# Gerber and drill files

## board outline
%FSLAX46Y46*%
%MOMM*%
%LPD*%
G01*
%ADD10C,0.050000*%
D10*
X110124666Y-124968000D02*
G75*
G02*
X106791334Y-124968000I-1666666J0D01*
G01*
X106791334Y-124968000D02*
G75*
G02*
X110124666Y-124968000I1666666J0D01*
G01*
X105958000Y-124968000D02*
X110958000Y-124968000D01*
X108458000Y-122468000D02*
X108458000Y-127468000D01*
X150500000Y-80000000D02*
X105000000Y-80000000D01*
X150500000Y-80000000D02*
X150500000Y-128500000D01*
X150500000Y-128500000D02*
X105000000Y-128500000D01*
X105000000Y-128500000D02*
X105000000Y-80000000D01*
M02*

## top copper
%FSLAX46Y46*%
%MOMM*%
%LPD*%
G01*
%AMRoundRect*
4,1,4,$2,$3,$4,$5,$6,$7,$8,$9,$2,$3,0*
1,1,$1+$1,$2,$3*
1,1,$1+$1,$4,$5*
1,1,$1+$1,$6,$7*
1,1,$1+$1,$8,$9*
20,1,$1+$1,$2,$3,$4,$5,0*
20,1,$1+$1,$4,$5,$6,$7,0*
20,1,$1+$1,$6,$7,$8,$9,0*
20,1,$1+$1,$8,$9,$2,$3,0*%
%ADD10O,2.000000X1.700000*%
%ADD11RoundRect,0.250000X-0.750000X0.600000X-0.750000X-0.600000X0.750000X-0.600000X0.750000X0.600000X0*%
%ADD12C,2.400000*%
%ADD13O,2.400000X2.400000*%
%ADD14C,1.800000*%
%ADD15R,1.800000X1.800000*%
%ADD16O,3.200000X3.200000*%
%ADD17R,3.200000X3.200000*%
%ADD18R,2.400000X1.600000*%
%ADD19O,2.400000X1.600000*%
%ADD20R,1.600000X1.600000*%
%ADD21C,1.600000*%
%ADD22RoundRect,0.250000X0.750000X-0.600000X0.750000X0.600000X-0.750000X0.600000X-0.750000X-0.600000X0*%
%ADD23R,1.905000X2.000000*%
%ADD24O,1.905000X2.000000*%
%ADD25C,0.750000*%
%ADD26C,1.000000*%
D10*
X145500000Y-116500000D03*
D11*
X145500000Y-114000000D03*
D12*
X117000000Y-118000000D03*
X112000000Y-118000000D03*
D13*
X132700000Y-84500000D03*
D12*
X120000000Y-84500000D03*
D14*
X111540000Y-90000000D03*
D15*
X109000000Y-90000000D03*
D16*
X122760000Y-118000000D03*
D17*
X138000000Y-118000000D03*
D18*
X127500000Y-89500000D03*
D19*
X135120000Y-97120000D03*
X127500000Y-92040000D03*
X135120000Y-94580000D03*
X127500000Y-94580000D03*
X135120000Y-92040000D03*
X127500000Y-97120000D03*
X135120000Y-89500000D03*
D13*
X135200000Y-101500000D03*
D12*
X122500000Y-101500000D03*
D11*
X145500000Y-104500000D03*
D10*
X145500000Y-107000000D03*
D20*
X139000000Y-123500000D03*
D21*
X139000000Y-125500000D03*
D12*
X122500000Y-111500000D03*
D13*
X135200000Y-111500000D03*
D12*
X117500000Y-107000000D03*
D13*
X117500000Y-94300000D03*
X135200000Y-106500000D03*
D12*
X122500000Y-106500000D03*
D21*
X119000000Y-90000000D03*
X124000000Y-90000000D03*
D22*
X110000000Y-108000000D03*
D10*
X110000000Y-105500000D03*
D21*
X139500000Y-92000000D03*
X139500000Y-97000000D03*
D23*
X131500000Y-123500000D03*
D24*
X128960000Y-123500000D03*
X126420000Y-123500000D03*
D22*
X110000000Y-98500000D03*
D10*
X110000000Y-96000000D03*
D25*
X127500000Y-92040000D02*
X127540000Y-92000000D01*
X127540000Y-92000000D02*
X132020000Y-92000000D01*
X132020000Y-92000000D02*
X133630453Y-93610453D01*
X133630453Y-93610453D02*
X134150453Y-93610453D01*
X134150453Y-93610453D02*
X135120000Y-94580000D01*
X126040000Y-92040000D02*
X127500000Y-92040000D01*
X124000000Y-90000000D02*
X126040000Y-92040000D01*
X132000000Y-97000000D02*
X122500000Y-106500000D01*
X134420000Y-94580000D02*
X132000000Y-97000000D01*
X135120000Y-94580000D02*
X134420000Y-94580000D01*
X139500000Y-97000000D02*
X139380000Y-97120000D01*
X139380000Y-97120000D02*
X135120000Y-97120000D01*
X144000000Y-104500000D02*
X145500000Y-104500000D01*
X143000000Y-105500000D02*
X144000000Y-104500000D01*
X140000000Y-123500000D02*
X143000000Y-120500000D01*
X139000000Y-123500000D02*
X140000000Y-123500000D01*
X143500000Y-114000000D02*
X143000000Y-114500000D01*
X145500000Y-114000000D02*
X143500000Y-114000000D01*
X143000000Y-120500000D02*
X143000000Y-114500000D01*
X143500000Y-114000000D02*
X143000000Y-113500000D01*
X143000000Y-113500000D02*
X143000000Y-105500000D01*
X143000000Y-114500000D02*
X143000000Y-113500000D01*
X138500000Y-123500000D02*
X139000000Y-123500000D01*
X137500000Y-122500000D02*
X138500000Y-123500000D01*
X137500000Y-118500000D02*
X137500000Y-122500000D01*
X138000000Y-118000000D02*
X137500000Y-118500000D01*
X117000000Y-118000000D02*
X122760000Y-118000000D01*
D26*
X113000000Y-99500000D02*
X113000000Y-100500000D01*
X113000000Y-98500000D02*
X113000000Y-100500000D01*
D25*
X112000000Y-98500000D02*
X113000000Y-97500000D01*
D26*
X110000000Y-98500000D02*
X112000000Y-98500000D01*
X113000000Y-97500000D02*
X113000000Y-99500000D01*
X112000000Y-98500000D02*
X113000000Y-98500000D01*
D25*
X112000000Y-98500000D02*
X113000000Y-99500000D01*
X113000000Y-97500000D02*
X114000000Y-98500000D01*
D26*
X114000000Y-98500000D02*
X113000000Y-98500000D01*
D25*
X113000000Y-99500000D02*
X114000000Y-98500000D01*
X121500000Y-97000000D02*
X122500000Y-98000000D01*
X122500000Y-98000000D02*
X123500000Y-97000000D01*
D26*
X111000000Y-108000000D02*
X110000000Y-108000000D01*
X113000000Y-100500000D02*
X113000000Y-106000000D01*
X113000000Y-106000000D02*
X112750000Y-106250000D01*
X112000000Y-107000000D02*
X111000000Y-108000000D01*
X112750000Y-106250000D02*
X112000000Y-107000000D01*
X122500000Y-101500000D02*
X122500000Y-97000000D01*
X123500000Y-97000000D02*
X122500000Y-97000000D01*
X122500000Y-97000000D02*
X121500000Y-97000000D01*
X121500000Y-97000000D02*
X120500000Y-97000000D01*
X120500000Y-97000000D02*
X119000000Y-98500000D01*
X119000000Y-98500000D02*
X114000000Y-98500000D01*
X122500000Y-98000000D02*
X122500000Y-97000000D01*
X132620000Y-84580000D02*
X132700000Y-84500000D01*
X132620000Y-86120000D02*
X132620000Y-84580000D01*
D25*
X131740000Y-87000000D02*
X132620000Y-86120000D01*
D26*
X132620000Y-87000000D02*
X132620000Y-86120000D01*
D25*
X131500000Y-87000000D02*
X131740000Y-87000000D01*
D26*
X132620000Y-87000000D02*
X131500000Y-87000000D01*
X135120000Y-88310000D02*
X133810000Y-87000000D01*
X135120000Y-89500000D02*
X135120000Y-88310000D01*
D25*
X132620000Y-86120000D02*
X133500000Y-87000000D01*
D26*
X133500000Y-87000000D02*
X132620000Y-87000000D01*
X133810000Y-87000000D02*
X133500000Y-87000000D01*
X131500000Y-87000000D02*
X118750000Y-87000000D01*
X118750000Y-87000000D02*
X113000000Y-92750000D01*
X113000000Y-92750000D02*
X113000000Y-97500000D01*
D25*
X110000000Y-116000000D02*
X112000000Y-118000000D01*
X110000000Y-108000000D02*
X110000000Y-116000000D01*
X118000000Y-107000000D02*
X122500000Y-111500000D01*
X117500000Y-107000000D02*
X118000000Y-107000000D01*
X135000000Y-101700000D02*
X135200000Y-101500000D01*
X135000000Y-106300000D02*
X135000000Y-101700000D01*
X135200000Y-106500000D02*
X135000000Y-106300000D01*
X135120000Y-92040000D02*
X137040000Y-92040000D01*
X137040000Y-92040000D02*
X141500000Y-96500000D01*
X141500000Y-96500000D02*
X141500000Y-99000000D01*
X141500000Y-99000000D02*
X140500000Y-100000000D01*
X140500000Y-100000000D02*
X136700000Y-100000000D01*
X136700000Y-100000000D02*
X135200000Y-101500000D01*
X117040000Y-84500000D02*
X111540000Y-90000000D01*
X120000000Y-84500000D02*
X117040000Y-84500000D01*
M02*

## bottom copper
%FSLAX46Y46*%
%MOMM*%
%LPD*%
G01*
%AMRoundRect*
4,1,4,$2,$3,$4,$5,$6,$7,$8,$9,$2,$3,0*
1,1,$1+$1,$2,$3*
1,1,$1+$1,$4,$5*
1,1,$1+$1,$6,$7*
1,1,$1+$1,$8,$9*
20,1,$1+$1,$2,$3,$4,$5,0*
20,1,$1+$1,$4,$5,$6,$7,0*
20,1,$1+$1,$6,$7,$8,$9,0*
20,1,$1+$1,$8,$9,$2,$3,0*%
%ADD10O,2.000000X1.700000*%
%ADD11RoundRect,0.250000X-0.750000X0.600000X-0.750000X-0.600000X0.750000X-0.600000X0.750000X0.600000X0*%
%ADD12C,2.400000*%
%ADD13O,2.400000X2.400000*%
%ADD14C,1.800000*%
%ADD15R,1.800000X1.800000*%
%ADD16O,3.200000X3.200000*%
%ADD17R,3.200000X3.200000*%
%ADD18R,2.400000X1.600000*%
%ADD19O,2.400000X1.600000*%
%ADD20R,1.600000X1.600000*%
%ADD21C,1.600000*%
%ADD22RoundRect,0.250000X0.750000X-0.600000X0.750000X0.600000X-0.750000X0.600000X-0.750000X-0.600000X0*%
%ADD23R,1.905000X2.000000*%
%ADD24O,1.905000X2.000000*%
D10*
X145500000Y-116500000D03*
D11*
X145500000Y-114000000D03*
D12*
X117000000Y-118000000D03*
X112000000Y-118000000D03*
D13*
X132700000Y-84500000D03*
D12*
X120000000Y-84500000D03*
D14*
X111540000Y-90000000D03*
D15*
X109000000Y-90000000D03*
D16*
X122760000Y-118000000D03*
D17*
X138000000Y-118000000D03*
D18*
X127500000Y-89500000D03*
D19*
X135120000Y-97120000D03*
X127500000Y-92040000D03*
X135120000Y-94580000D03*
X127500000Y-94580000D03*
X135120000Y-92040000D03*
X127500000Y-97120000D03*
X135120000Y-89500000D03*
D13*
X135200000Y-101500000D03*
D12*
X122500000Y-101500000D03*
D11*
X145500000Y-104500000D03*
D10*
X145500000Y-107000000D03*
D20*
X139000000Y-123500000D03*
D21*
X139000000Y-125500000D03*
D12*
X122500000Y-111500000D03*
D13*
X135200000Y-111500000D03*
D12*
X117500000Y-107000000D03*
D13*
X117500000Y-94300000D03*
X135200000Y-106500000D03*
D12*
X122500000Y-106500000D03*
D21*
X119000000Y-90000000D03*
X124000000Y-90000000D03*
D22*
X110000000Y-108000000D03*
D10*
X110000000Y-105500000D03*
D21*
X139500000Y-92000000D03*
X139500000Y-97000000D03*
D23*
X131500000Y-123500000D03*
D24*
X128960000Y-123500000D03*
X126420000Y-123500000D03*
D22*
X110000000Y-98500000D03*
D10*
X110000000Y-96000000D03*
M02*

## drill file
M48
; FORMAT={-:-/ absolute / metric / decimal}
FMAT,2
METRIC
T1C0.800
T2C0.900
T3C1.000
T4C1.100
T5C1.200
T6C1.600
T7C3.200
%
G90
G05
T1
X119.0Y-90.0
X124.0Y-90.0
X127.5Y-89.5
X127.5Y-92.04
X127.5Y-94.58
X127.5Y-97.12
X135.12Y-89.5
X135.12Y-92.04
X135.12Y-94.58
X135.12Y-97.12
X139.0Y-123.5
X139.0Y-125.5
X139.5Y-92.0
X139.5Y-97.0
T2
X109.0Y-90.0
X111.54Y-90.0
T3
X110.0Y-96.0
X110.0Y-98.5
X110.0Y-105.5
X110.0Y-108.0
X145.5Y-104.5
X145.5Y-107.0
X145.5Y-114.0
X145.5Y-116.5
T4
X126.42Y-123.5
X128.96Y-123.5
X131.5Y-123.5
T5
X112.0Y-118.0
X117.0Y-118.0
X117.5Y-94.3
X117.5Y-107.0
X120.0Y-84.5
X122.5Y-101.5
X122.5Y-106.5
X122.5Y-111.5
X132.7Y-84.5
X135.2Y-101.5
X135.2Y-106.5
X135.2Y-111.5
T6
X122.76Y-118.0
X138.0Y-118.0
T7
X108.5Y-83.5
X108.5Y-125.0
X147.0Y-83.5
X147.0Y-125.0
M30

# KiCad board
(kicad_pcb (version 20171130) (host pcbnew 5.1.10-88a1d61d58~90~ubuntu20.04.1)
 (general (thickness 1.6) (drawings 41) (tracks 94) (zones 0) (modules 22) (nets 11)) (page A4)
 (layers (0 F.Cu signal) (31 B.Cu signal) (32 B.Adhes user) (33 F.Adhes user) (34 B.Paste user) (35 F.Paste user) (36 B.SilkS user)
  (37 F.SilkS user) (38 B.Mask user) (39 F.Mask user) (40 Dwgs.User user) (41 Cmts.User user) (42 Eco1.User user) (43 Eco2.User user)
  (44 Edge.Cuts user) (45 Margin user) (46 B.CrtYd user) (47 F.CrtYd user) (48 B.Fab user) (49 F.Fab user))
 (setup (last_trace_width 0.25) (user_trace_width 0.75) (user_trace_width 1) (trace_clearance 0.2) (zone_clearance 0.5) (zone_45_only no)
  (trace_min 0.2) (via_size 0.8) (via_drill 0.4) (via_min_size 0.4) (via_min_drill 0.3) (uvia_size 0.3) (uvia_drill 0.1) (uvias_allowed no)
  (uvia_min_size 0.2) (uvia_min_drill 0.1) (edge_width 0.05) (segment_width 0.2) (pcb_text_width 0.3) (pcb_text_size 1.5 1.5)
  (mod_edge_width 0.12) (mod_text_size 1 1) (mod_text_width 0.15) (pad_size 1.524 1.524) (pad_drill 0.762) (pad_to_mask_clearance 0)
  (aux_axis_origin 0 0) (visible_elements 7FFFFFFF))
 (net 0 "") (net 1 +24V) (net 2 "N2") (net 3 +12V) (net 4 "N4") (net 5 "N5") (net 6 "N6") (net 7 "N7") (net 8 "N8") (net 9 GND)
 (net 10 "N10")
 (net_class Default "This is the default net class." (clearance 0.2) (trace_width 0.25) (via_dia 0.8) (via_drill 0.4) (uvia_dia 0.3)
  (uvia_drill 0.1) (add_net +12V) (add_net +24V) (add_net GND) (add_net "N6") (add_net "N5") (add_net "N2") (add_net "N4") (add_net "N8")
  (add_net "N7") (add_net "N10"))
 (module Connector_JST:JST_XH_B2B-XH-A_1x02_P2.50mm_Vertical (layer F.Cu) (at 145.5 114 270)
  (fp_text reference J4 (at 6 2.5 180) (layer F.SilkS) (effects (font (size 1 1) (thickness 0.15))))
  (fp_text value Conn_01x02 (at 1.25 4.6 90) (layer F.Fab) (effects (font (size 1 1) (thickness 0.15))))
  (pad 2 thru_hole oval (at 2.5 0 270) (size 1.7 2) (drill 1) (layers *.Cu *.Mask))
  (pad 1 thru_hole roundrect (at 0 0 270) (size 1.7 2) (drill 1) (layers *.Cu *.Mask) (roundrect_rratio 0.1470588235294118) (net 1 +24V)))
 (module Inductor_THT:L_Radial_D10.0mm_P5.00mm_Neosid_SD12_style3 (layer F.Cu) (at 112 118)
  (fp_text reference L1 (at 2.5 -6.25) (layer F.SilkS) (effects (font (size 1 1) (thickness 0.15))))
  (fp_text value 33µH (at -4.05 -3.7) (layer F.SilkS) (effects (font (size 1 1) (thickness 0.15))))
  (pad 2 thru_hole circle (at 5 0) (size 2.4 2.4) (drill 1.2) (layers *.Cu *.Mask) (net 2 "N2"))
  (pad 1 thru_hole circle (at 0 0) (size 2.4 2.4) (drill 1.2) (layers *.Cu *.Mask) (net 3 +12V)))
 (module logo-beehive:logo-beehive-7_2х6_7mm (layer F.Cu) (at 139 85)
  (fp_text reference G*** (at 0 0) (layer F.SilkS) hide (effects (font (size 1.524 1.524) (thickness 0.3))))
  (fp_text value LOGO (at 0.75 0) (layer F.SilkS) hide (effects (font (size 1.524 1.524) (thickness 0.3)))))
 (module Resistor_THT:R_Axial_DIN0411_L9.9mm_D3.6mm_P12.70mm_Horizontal (layer F.Cu) (at 120 84.5)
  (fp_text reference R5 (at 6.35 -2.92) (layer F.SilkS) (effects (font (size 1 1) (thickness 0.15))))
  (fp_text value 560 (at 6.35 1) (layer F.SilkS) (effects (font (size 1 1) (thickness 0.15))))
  (pad 2 thru_hole oval (at 12.7 0) (size 2.4 2.4) (drill 1.2) (layers *.Cu *.Mask) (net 3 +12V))
  (pad 1 thru_hole circle (at 0 0) (size 2.4 2.4) (drill 1.2) (layers *.Cu *.Mask) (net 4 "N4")))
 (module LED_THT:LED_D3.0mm (layer F.Cu) (at 109 90)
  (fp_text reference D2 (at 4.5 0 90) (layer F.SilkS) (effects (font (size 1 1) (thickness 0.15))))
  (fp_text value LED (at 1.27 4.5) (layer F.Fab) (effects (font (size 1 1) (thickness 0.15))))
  (pad 2 thru_hole circle (at 2.54 0) (size 1.8 1.8) (drill 0.9) (layers *.Cu *.Mask) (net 4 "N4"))
  (pad 1 thru_hole rect (at 0 0) (size 1.8 1.8) (drill 0.9) (layers *.Cu *.Mask)))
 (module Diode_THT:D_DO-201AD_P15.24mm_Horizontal (layer F.Cu) (at 138 118 180)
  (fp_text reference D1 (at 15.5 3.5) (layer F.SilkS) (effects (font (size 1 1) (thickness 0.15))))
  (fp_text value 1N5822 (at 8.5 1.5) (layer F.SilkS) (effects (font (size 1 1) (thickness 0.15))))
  (pad 2 thru_hole oval (at 15.24 0 180) (size 3.2 3.2) (drill 1.6) (layers *.Cu *.Mask) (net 2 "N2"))
  (pad 1 thru_hole rect (at 0 0 180) (size 3.2 3.2) (drill 1.6) (layers *.Cu *.Mask) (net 1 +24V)))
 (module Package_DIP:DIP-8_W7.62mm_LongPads (layer F.Cu) (at 127.5 89.5)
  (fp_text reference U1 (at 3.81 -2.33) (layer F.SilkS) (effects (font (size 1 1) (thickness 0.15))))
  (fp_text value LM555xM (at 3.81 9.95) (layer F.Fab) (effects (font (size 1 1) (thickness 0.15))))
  (pad 1 thru_hole rect (at 0 0) (size 2.4 1.6) (drill 0.8) (layers *.Cu *.Mask))
  (pad 5 thru_hole oval (at 7.62 7.62) (size 2.4 1.6) (drill 0.8) (layers *.Cu *.Mask) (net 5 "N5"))
  (pad 2 thru_hole oval (at 0 2.54) (size 2.4 1.6) (drill 0.8) (layers *.Cu *.Mask) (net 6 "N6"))
  (pad 6 thru_hole oval (at 7.62 5.08) (size 2.4 1.6) (drill 0.8) (layers *.Cu *.Mask) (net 6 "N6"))
  (pad 3 thru_hole oval (at 0 5.08) (size 2.4 1.6) (drill 0.8) (layers *.Cu *.Mask))
  (pad 7 thru_hole oval (at 7.62 2.54) (size 2.4 1.6) (drill 0.8) (layers *.Cu *.Mask) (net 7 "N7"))
  (pad 4 thru_hole oval (at 0 7.62) (size 2.4 1.6) (drill 0.8) (layers *.Cu *.Mask))
  (pad 8 thru_hole oval (at 7.62 0) (size 2.4 1.6) (drill 0.8) (layers *.Cu *.Mask) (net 3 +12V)))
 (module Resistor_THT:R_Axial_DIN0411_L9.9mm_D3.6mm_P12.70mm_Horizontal (layer F.Cu) (at 122.5 101.5)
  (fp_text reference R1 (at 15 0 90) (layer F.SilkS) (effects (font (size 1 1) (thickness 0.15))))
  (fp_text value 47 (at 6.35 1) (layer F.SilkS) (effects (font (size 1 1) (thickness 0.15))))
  (pad 2 thru_hole oval (at 12.7 0) (size 2.4 2.4) (drill 1.2) (layers *.Cu *.Mask) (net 7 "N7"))
  (pad 1 thru_hole circle (at 0 0) (size 2.4 2.4) (drill 1.2) (layers *.Cu *.Mask) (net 3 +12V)))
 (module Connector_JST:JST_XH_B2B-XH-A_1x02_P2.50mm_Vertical (layer F.Cu) (at 145.5 104.5 270)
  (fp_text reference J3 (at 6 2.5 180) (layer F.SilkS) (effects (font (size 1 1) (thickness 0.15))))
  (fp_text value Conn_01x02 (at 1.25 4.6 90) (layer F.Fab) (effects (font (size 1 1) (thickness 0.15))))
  (pad 1 thru_hole roundrect (at 0 0 270) (size 1.7 2) (drill 1) (layers *.Cu *.Mask) (roundrect_rratio 0.1470588235294118) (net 1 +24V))
  (pad 2 thru_hole oval (at 2.5 0 270) (size 1.7 2) (drill 1) (layers *.Cu *.Mask)))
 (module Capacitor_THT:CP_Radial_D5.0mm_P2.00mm (layer F.Cu) (at 139 123.5 270)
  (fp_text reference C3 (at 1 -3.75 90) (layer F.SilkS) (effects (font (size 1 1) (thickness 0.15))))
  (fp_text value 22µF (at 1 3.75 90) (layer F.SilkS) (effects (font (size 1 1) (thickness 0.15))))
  (pad 1 thru_hole rect (at 0 0 270) (size 1.6 1.6) (drill 0.8) (layers *.Cu *.Mask) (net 1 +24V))
  (pad 2 thru_hole circle (at 2 0 270) (size 1.6 1.6) (drill 0.8) (layers *.Cu *.Mask)))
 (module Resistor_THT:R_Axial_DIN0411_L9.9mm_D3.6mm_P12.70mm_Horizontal (layer F.Cu) (at 122.5 111.5)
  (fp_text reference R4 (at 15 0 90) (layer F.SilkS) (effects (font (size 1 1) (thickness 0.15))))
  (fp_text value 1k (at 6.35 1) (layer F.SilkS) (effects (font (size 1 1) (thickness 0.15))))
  (pad 1 thru_hole circle (at 0 0) (size 2.4 2.4) (drill 1.2) (layers *.Cu *.Mask) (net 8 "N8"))
  (pad 2 thru_hole oval (at 12.7 0) (size 2.4 2.4) (drill 1.2) (layers *.Cu *.Mask)))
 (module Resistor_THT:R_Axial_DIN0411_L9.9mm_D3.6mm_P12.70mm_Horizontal (layer F.Cu) (at 117.5 107 90)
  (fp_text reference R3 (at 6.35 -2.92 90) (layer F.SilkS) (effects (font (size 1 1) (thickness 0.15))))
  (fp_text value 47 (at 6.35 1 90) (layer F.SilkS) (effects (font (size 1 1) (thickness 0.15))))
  (pad 1 thru_hole circle (at 0 0 90) (size 2.4 2.4) (drill 1.2) (layers *.Cu *.Mask) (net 8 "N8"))
  (pad 2 thru_hole oval (at 12.7 0 90) (size 2.4 2.4) (drill 1.2) (layers *.Cu *.Mask)))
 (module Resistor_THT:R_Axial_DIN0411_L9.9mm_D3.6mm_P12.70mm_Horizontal (layer F.Cu) (at 122.5 106.5)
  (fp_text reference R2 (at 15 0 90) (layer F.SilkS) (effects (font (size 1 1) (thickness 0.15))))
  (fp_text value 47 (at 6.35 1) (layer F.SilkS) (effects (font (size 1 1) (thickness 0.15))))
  (pad 2 thru_hole oval (at 12.7 0) (size 2.4 2.4) (drill 1.2) (layers *.Cu *.Mask) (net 7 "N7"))
  (pad 1 thru_hole circle (at 0 0) (size 2.4 2.4) (drill 1.2) (layers *.Cu *.Mask) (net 6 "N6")))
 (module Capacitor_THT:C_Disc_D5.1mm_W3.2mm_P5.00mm (layer F.Cu) (at 119 90)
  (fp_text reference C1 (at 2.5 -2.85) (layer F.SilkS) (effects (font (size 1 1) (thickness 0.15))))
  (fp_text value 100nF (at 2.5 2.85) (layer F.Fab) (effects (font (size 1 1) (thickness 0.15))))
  (pad 1 thru_hole circle (at 0 0) (size 1.6 1.6) (drill 0.8) (layers *.Cu *.Mask))
  (pad 2 thru_hole circle (at 5 0) (size 1.6 1.6) (drill 0.8) (layers *.Cu *.Mask) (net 6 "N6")))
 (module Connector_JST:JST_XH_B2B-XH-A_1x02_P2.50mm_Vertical (layer F.Cu) (at 110 108 90)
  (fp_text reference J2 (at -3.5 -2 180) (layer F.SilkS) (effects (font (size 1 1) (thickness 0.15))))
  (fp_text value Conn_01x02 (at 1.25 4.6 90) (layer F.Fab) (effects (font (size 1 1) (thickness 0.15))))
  (pad 1 thru_hole roundrect (at 0 0 90) (size 1.7 2) (drill 1) (layers *.Cu *.Mask) (roundrect_rratio 0.1470588235294118) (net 3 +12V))
  (pad 2 thru_hole oval (at 2.5 0 90) (size 1.7 2) (drill 1) (layers *.Cu *.Mask)))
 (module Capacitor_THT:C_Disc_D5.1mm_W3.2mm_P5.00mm (layer F.Cu) (at 139.5 92 270)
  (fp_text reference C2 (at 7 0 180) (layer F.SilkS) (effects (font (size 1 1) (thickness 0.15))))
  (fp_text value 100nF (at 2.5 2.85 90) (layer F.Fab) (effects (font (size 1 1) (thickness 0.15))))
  (pad 1 thru_hole circle (at 0 0 270) (size 1.6 1.6) (drill 0.8) (layers *.Cu *.Mask))
  (pad 2 thru_hole circle (at 5 0 270) (size 1.6 1.6) (drill 0.8) (layers *.Cu *.Mask) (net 5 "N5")))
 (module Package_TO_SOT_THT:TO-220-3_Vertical (layer F.Cu) (at 131.5 123.5 180)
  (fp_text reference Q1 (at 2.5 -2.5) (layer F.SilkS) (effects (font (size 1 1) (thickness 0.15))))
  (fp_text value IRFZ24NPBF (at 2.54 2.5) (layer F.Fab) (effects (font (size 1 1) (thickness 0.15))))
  (pad 1 thru_hole rect (at 0 0 180) (size 1.905 2) (drill 1.1) (layers *.Cu *.Mask))
  (pad 2 thru_hole oval (at 2.54 0 180) (size 1.905 2) (drill 1.1) (layers *.Cu *.Mask))
  (pad 3 thru_hole oval (at 5.08 0 180) (size 1.905 2) (drill 1.1) (layers *.Cu *.Mask)))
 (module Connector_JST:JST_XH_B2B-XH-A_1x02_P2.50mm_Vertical (layer F.Cu) (at 110 98.5 90)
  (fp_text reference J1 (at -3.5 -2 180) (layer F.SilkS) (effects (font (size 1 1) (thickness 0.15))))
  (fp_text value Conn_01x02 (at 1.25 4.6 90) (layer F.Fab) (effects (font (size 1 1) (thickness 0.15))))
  (pad 1 thru_hole roundrect (at 0 0 90) (size 1.7 2) (drill 1) (layers *.Cu *.Mask) (roundrect_rratio 0.1470588235294118) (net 3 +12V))
  (pad 2 thru_hole oval (at 2.5 0 90) (size 1.7 2) (drill 1) (layers *.Cu *.Mask)))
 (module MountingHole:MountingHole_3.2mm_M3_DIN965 (layer F.Cu) (at 147 83.5)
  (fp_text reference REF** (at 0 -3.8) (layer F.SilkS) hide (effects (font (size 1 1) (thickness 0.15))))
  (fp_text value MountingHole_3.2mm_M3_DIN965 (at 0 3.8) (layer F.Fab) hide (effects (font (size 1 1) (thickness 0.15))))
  (pad 1 np_thru_hole circle (at 0 0) (size 3.2 3.2) (drill 3.2) (layers *.Cu *.Mask)))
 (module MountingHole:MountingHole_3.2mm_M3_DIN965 (layer F.Cu) (at 108.5 125)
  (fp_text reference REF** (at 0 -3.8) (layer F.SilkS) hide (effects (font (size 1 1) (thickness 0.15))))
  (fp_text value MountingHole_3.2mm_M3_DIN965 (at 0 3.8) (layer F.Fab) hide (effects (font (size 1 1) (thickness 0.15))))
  (pad 1 np_thru_hole circle (at 0 0) (size 3.2 3.2) (drill 3.2) (layers *.Cu *.Mask)))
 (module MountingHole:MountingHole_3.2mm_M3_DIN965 (layer F.Cu) (at 147 125)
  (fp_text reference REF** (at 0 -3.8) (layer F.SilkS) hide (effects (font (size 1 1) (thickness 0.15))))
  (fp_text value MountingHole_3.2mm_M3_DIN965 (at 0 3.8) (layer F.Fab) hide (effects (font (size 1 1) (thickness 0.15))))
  (pad 1 np_thru_hole circle (at 0 0) (size 3.2 3.2) (drill 3.2) (layers *.Cu *.Mask)))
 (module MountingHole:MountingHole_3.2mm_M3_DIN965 (layer F.Cu) (at 108.5 83.5)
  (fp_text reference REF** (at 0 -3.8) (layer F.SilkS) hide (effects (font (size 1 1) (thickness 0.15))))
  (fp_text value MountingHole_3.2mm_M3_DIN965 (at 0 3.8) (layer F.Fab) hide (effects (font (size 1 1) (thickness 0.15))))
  (pad 1 np_thru_hole circle (at 0 0) (size 3.2 3.2) (drill 3.2) (layers *.Cu *.Mask)))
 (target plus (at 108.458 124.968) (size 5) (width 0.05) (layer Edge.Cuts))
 (gr_line (start 150.5 80) (end 105 80) (layer Edge.Cuts) (width 0.05))
 (gr_line (start 150.5 80) (end 150.5 128.5) (layer Edge.Cuts) (width 0.05))
 (gr_line (start 150.5 128.5) (end 105 128.5) (layer Edge.Cuts) (width 0.05))
 (gr_line (start 105 128.5) (end 105 80) (layer Edge.Cuts) (width 0.05))
 (segment (start 127.5 92.04) (end 127.54 92) (width 0.75) (layer F.Cu) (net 6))
 (segment (start 127.54 92) (end 132.02 92) (width 0.75) (layer F.Cu) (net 6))
 (segment (start 132.02 92) (end 133.630453 93.610453) (width 0.75) (layer F.Cu) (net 6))
 (segment (start 133.630453 93.610453) (end 134.150453 93.610453) (width 0.75) (layer F.Cu) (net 6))
 (segment (start 134.150453 93.610453) (end 135.12 94.58) (width 0.75) (layer F.Cu) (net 6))
 (segment (start 126.04 92.04) (end 127.5 92.04) (width 0.75) (layer F.Cu) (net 6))
 (segment (start 124 90) (end 126.04 92.04) (width 0.75) (layer F.Cu) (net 6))
 (segment (start 132 97) (end 122.5 106.5) (width 0.75) (layer F.Cu) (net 6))
 (segment (start 134.42 94.58) (end 132 97) (width 0.75) (layer F.Cu) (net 6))
 (segment (start 135.12 94.58) (end 134.42 94.58) (width 0.75) (layer F.Cu) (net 6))
 (segment (start 139.5 97) (end 139.38 97.12) (width 0.75) (layer F.Cu) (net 5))
 (segment (start 139.38 97.12) (end 135.12 97.12) (width 0.75) (layer F.Cu) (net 5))
 (segment (start 144 104.5) (end 145.5 104.5) (width 0.75) (layer F.Cu) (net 1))
 (segment (start 143 105.5) (end 144 104.5) (width 0.75) (layer F.Cu) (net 1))
 (segment (start 140 123.5) (end 143 120.5) (width 0.75) (layer F.Cu) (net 1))
 (segment (start 139 123.5) (end 140 123.5) (width 0.75) (layer F.Cu) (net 1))
 (segment (start 143.5 114) (end 143 114.5) (width 0.75) (layer F.Cu) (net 1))
 (segment (start 145.5 114) (end 143.5 114) (width 0.75) (layer F.Cu) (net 1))
 (segment (start 143 120.5) (end 143 114.5) (width 0.75) (layer F.Cu) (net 1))
 (segment (start 143.5 114) (end 143 113.5) (width 0.75) (layer F.Cu) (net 1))
 (segment (start 143 113.5) (end 143 105.5) (width 0.75) (layer F.Cu) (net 1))
 (segment (start 143 114.5) (end 143 113.5) (width 0.75) (layer F.Cu) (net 1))
 (segment (start 138.5 123.5) (end 139 123.5) (width 0.75) (layer F.Cu) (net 1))
 (segment (start 137.5 122.5) (end 138.5 123.5) (width 0.75) (layer F.Cu) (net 1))
 (segment (start 137.5 118.5) (end 137.5 122.5) (width 0.75) (layer F.Cu) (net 1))
 (segment (start 138 118) (end 137.5 118.5) (width 0.75) (layer F.Cu) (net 1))
 (segment (start 117 118) (end 122.76 118) (width 0.75) (layer F.Cu) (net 2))
 (segment (start 113 99.5) (end 113 100.5) (width 1) (layer F.Cu) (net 3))
 (segment (start 113 98.5) (end 113 100.5) (width 1) (layer F.Cu) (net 3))
 (segment (start 112 98.5) (end 113 97.5) (width 0.75) (layer F.Cu) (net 3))
 (segment (start 110 98.5) (end 112 98.5) (width 1) (layer F.Cu) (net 3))
 (segment (start 113 97.5) (end 113 99.5) (width 1) (layer F.Cu) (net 3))
 (segment (start 112 98.5) (end 113 98.5) (width 1) (layer F.Cu) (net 3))
 (segment (start 112 98.5) (end 113 99.5) (width 0.75) (layer F.Cu) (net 3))
 (segment (start 113 97.5) (end 114 98.5) (width 0.75) (layer F.Cu) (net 3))
 (segment (start 114 98.5) (end 113 98.5) (width 1) (layer F.Cu) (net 3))
 (segment (start 113 99.5) (end 114 98.5) (width 0.75) (layer F.Cu) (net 3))
 (segment (start 121.5 97) (end 122.5 98) (width 0.75) (layer F.Cu) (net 3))
 (segment (start 122.5 98) (end 123.5 97) (width 0.75) (layer F.Cu) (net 3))
 (segment (start 111 108) (end 110 108) (width 1) (layer F.Cu) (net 3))
 (segment (start 113 100.5) (end 113 106) (width 1) (layer F.Cu) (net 3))
 (segment (start 113 106) (end 112.75 106.25) (width 1) (layer F.Cu) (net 3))
 (segment (start 112 107) (end 111 108) (width 1) (layer F.Cu) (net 3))
 (segment (start 112.75 106.25) (end 112 107) (width 1) (layer F.Cu) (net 3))
 (segment (start 122.5 101.5) (end 122.5 97) (width 1) (layer F.Cu) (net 3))
 (segment (start 123.5 97) (end 122.5 97) (width 1) (layer F.Cu) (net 3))
 (segment (start 122.5 97) (end 121.5 97) (width 1) (layer F.Cu) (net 3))
 (segment (start 121.5 97) (end 120.5 97) (width 1) (layer F.Cu) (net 3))
 (segment (start 120.5 97) (end 119 98.5) (width 1) (layer F.Cu) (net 3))
 (segment (start 119 98.5) (end 114 98.5) (width 1) (layer F.Cu) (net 3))
 (segment (start 122.5 98) (end 122.5 97) (width 1) (layer F.Cu) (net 3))
 (segment (start 132.62 84.58) (end 132.7 84.5) (width 1) (layer F.Cu) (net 3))
 (segment (start 132.62 86.12) (end 132.62 84.58) (width 1) (layer F.Cu) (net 3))
 (segment (start 131.74 87) (end 132.62 86.12) (width 0.75) (layer F.Cu) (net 3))
 (segment (start 132.62 87) (end 132.62 86.12) (width 1) (layer F.Cu) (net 3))
 (segment (start 131.5 87) (end 131.74 87) (width 0.75) (layer F.Cu) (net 3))
 (segment (start 132.62 87) (end 131.5 87) (width 1) (layer F.Cu) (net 3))
 (segment (start 135.12 88.31) (end 133.81 87) (width 1) (layer F.Cu) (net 3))
 (segment (start 135.12 89.5) (end 135.12 88.31) (width 1) (layer F.Cu) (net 3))
 (segment (start 132.62 86.12) (end 133.5 87) (width 0.75) (layer F.Cu) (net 3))
 (segment (start 133.5 87) (end 132.62 87) (width 1) (layer F.Cu) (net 3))
 (segment (start 133.81 87) (end 133.5 87) (width 1) (layer F.Cu) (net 3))
 (segment (start 131.5 87) (end 118.75 87) (width 1) (layer F.Cu) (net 3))
 (segment (start 118.75 87) (end 113 92.75) (width 1) (layer F.Cu) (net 3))
 (segment (start 113 92.75) (end 113 97.5) (width 1) (layer F.Cu) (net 3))
 (segment (start 110 116) (end 112 118) (width 0.75) (layer F.Cu) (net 3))
 (segment (start 110 108) (end 110 116) (width 0.75) (layer F.Cu) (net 3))
 (segment (start 118 107) (end 122.5 111.5) (width 0.75) (layer F.Cu) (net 8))
 (segment (start 117.5 107) (end 118 107) (width 0.75) (layer F.Cu) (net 8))
 (segment (start 135 101.7) (end 135.2 101.5) (width 0.75) (layer F.Cu) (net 7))
 (segment (start 135 106.3) (end 135 101.7) (width 0.75) (layer F.Cu) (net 7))
 (segment (start 135.2 106.5) (end 135 106.3) (width 0.75) (layer F.Cu) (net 7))
 (segment (start 135.12 92.04) (end 137.04 92.04) (width 0.75) (layer F.Cu) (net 7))
 (segment (start 137.04 92.04) (end 141.5 96.5) (width 0.75) (layer F.Cu) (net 7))
 (segment (start 141.5 96.5) (end 141.5 99) (width 0.75) (layer F.Cu) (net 7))
 (segment (start 141.5 99) (end 140.5 100) (width 0.75) (layer F.Cu) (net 7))
 (segment (start 140.5 100) (end 136.7 100) (width 0.75) (layer F.Cu) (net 7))
 (segment (start 136.7 100) (end 135.2 101.5) (width 0.75) (layer F.Cu) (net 7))
 (segment (start 117.04 84.5) (end 111.54 90) (width 0.75) (layer F.Cu) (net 4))
 (segment (start 120 84.5) (end 117.04 84.5) (width 0.75) (layer F.Cu) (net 4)))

